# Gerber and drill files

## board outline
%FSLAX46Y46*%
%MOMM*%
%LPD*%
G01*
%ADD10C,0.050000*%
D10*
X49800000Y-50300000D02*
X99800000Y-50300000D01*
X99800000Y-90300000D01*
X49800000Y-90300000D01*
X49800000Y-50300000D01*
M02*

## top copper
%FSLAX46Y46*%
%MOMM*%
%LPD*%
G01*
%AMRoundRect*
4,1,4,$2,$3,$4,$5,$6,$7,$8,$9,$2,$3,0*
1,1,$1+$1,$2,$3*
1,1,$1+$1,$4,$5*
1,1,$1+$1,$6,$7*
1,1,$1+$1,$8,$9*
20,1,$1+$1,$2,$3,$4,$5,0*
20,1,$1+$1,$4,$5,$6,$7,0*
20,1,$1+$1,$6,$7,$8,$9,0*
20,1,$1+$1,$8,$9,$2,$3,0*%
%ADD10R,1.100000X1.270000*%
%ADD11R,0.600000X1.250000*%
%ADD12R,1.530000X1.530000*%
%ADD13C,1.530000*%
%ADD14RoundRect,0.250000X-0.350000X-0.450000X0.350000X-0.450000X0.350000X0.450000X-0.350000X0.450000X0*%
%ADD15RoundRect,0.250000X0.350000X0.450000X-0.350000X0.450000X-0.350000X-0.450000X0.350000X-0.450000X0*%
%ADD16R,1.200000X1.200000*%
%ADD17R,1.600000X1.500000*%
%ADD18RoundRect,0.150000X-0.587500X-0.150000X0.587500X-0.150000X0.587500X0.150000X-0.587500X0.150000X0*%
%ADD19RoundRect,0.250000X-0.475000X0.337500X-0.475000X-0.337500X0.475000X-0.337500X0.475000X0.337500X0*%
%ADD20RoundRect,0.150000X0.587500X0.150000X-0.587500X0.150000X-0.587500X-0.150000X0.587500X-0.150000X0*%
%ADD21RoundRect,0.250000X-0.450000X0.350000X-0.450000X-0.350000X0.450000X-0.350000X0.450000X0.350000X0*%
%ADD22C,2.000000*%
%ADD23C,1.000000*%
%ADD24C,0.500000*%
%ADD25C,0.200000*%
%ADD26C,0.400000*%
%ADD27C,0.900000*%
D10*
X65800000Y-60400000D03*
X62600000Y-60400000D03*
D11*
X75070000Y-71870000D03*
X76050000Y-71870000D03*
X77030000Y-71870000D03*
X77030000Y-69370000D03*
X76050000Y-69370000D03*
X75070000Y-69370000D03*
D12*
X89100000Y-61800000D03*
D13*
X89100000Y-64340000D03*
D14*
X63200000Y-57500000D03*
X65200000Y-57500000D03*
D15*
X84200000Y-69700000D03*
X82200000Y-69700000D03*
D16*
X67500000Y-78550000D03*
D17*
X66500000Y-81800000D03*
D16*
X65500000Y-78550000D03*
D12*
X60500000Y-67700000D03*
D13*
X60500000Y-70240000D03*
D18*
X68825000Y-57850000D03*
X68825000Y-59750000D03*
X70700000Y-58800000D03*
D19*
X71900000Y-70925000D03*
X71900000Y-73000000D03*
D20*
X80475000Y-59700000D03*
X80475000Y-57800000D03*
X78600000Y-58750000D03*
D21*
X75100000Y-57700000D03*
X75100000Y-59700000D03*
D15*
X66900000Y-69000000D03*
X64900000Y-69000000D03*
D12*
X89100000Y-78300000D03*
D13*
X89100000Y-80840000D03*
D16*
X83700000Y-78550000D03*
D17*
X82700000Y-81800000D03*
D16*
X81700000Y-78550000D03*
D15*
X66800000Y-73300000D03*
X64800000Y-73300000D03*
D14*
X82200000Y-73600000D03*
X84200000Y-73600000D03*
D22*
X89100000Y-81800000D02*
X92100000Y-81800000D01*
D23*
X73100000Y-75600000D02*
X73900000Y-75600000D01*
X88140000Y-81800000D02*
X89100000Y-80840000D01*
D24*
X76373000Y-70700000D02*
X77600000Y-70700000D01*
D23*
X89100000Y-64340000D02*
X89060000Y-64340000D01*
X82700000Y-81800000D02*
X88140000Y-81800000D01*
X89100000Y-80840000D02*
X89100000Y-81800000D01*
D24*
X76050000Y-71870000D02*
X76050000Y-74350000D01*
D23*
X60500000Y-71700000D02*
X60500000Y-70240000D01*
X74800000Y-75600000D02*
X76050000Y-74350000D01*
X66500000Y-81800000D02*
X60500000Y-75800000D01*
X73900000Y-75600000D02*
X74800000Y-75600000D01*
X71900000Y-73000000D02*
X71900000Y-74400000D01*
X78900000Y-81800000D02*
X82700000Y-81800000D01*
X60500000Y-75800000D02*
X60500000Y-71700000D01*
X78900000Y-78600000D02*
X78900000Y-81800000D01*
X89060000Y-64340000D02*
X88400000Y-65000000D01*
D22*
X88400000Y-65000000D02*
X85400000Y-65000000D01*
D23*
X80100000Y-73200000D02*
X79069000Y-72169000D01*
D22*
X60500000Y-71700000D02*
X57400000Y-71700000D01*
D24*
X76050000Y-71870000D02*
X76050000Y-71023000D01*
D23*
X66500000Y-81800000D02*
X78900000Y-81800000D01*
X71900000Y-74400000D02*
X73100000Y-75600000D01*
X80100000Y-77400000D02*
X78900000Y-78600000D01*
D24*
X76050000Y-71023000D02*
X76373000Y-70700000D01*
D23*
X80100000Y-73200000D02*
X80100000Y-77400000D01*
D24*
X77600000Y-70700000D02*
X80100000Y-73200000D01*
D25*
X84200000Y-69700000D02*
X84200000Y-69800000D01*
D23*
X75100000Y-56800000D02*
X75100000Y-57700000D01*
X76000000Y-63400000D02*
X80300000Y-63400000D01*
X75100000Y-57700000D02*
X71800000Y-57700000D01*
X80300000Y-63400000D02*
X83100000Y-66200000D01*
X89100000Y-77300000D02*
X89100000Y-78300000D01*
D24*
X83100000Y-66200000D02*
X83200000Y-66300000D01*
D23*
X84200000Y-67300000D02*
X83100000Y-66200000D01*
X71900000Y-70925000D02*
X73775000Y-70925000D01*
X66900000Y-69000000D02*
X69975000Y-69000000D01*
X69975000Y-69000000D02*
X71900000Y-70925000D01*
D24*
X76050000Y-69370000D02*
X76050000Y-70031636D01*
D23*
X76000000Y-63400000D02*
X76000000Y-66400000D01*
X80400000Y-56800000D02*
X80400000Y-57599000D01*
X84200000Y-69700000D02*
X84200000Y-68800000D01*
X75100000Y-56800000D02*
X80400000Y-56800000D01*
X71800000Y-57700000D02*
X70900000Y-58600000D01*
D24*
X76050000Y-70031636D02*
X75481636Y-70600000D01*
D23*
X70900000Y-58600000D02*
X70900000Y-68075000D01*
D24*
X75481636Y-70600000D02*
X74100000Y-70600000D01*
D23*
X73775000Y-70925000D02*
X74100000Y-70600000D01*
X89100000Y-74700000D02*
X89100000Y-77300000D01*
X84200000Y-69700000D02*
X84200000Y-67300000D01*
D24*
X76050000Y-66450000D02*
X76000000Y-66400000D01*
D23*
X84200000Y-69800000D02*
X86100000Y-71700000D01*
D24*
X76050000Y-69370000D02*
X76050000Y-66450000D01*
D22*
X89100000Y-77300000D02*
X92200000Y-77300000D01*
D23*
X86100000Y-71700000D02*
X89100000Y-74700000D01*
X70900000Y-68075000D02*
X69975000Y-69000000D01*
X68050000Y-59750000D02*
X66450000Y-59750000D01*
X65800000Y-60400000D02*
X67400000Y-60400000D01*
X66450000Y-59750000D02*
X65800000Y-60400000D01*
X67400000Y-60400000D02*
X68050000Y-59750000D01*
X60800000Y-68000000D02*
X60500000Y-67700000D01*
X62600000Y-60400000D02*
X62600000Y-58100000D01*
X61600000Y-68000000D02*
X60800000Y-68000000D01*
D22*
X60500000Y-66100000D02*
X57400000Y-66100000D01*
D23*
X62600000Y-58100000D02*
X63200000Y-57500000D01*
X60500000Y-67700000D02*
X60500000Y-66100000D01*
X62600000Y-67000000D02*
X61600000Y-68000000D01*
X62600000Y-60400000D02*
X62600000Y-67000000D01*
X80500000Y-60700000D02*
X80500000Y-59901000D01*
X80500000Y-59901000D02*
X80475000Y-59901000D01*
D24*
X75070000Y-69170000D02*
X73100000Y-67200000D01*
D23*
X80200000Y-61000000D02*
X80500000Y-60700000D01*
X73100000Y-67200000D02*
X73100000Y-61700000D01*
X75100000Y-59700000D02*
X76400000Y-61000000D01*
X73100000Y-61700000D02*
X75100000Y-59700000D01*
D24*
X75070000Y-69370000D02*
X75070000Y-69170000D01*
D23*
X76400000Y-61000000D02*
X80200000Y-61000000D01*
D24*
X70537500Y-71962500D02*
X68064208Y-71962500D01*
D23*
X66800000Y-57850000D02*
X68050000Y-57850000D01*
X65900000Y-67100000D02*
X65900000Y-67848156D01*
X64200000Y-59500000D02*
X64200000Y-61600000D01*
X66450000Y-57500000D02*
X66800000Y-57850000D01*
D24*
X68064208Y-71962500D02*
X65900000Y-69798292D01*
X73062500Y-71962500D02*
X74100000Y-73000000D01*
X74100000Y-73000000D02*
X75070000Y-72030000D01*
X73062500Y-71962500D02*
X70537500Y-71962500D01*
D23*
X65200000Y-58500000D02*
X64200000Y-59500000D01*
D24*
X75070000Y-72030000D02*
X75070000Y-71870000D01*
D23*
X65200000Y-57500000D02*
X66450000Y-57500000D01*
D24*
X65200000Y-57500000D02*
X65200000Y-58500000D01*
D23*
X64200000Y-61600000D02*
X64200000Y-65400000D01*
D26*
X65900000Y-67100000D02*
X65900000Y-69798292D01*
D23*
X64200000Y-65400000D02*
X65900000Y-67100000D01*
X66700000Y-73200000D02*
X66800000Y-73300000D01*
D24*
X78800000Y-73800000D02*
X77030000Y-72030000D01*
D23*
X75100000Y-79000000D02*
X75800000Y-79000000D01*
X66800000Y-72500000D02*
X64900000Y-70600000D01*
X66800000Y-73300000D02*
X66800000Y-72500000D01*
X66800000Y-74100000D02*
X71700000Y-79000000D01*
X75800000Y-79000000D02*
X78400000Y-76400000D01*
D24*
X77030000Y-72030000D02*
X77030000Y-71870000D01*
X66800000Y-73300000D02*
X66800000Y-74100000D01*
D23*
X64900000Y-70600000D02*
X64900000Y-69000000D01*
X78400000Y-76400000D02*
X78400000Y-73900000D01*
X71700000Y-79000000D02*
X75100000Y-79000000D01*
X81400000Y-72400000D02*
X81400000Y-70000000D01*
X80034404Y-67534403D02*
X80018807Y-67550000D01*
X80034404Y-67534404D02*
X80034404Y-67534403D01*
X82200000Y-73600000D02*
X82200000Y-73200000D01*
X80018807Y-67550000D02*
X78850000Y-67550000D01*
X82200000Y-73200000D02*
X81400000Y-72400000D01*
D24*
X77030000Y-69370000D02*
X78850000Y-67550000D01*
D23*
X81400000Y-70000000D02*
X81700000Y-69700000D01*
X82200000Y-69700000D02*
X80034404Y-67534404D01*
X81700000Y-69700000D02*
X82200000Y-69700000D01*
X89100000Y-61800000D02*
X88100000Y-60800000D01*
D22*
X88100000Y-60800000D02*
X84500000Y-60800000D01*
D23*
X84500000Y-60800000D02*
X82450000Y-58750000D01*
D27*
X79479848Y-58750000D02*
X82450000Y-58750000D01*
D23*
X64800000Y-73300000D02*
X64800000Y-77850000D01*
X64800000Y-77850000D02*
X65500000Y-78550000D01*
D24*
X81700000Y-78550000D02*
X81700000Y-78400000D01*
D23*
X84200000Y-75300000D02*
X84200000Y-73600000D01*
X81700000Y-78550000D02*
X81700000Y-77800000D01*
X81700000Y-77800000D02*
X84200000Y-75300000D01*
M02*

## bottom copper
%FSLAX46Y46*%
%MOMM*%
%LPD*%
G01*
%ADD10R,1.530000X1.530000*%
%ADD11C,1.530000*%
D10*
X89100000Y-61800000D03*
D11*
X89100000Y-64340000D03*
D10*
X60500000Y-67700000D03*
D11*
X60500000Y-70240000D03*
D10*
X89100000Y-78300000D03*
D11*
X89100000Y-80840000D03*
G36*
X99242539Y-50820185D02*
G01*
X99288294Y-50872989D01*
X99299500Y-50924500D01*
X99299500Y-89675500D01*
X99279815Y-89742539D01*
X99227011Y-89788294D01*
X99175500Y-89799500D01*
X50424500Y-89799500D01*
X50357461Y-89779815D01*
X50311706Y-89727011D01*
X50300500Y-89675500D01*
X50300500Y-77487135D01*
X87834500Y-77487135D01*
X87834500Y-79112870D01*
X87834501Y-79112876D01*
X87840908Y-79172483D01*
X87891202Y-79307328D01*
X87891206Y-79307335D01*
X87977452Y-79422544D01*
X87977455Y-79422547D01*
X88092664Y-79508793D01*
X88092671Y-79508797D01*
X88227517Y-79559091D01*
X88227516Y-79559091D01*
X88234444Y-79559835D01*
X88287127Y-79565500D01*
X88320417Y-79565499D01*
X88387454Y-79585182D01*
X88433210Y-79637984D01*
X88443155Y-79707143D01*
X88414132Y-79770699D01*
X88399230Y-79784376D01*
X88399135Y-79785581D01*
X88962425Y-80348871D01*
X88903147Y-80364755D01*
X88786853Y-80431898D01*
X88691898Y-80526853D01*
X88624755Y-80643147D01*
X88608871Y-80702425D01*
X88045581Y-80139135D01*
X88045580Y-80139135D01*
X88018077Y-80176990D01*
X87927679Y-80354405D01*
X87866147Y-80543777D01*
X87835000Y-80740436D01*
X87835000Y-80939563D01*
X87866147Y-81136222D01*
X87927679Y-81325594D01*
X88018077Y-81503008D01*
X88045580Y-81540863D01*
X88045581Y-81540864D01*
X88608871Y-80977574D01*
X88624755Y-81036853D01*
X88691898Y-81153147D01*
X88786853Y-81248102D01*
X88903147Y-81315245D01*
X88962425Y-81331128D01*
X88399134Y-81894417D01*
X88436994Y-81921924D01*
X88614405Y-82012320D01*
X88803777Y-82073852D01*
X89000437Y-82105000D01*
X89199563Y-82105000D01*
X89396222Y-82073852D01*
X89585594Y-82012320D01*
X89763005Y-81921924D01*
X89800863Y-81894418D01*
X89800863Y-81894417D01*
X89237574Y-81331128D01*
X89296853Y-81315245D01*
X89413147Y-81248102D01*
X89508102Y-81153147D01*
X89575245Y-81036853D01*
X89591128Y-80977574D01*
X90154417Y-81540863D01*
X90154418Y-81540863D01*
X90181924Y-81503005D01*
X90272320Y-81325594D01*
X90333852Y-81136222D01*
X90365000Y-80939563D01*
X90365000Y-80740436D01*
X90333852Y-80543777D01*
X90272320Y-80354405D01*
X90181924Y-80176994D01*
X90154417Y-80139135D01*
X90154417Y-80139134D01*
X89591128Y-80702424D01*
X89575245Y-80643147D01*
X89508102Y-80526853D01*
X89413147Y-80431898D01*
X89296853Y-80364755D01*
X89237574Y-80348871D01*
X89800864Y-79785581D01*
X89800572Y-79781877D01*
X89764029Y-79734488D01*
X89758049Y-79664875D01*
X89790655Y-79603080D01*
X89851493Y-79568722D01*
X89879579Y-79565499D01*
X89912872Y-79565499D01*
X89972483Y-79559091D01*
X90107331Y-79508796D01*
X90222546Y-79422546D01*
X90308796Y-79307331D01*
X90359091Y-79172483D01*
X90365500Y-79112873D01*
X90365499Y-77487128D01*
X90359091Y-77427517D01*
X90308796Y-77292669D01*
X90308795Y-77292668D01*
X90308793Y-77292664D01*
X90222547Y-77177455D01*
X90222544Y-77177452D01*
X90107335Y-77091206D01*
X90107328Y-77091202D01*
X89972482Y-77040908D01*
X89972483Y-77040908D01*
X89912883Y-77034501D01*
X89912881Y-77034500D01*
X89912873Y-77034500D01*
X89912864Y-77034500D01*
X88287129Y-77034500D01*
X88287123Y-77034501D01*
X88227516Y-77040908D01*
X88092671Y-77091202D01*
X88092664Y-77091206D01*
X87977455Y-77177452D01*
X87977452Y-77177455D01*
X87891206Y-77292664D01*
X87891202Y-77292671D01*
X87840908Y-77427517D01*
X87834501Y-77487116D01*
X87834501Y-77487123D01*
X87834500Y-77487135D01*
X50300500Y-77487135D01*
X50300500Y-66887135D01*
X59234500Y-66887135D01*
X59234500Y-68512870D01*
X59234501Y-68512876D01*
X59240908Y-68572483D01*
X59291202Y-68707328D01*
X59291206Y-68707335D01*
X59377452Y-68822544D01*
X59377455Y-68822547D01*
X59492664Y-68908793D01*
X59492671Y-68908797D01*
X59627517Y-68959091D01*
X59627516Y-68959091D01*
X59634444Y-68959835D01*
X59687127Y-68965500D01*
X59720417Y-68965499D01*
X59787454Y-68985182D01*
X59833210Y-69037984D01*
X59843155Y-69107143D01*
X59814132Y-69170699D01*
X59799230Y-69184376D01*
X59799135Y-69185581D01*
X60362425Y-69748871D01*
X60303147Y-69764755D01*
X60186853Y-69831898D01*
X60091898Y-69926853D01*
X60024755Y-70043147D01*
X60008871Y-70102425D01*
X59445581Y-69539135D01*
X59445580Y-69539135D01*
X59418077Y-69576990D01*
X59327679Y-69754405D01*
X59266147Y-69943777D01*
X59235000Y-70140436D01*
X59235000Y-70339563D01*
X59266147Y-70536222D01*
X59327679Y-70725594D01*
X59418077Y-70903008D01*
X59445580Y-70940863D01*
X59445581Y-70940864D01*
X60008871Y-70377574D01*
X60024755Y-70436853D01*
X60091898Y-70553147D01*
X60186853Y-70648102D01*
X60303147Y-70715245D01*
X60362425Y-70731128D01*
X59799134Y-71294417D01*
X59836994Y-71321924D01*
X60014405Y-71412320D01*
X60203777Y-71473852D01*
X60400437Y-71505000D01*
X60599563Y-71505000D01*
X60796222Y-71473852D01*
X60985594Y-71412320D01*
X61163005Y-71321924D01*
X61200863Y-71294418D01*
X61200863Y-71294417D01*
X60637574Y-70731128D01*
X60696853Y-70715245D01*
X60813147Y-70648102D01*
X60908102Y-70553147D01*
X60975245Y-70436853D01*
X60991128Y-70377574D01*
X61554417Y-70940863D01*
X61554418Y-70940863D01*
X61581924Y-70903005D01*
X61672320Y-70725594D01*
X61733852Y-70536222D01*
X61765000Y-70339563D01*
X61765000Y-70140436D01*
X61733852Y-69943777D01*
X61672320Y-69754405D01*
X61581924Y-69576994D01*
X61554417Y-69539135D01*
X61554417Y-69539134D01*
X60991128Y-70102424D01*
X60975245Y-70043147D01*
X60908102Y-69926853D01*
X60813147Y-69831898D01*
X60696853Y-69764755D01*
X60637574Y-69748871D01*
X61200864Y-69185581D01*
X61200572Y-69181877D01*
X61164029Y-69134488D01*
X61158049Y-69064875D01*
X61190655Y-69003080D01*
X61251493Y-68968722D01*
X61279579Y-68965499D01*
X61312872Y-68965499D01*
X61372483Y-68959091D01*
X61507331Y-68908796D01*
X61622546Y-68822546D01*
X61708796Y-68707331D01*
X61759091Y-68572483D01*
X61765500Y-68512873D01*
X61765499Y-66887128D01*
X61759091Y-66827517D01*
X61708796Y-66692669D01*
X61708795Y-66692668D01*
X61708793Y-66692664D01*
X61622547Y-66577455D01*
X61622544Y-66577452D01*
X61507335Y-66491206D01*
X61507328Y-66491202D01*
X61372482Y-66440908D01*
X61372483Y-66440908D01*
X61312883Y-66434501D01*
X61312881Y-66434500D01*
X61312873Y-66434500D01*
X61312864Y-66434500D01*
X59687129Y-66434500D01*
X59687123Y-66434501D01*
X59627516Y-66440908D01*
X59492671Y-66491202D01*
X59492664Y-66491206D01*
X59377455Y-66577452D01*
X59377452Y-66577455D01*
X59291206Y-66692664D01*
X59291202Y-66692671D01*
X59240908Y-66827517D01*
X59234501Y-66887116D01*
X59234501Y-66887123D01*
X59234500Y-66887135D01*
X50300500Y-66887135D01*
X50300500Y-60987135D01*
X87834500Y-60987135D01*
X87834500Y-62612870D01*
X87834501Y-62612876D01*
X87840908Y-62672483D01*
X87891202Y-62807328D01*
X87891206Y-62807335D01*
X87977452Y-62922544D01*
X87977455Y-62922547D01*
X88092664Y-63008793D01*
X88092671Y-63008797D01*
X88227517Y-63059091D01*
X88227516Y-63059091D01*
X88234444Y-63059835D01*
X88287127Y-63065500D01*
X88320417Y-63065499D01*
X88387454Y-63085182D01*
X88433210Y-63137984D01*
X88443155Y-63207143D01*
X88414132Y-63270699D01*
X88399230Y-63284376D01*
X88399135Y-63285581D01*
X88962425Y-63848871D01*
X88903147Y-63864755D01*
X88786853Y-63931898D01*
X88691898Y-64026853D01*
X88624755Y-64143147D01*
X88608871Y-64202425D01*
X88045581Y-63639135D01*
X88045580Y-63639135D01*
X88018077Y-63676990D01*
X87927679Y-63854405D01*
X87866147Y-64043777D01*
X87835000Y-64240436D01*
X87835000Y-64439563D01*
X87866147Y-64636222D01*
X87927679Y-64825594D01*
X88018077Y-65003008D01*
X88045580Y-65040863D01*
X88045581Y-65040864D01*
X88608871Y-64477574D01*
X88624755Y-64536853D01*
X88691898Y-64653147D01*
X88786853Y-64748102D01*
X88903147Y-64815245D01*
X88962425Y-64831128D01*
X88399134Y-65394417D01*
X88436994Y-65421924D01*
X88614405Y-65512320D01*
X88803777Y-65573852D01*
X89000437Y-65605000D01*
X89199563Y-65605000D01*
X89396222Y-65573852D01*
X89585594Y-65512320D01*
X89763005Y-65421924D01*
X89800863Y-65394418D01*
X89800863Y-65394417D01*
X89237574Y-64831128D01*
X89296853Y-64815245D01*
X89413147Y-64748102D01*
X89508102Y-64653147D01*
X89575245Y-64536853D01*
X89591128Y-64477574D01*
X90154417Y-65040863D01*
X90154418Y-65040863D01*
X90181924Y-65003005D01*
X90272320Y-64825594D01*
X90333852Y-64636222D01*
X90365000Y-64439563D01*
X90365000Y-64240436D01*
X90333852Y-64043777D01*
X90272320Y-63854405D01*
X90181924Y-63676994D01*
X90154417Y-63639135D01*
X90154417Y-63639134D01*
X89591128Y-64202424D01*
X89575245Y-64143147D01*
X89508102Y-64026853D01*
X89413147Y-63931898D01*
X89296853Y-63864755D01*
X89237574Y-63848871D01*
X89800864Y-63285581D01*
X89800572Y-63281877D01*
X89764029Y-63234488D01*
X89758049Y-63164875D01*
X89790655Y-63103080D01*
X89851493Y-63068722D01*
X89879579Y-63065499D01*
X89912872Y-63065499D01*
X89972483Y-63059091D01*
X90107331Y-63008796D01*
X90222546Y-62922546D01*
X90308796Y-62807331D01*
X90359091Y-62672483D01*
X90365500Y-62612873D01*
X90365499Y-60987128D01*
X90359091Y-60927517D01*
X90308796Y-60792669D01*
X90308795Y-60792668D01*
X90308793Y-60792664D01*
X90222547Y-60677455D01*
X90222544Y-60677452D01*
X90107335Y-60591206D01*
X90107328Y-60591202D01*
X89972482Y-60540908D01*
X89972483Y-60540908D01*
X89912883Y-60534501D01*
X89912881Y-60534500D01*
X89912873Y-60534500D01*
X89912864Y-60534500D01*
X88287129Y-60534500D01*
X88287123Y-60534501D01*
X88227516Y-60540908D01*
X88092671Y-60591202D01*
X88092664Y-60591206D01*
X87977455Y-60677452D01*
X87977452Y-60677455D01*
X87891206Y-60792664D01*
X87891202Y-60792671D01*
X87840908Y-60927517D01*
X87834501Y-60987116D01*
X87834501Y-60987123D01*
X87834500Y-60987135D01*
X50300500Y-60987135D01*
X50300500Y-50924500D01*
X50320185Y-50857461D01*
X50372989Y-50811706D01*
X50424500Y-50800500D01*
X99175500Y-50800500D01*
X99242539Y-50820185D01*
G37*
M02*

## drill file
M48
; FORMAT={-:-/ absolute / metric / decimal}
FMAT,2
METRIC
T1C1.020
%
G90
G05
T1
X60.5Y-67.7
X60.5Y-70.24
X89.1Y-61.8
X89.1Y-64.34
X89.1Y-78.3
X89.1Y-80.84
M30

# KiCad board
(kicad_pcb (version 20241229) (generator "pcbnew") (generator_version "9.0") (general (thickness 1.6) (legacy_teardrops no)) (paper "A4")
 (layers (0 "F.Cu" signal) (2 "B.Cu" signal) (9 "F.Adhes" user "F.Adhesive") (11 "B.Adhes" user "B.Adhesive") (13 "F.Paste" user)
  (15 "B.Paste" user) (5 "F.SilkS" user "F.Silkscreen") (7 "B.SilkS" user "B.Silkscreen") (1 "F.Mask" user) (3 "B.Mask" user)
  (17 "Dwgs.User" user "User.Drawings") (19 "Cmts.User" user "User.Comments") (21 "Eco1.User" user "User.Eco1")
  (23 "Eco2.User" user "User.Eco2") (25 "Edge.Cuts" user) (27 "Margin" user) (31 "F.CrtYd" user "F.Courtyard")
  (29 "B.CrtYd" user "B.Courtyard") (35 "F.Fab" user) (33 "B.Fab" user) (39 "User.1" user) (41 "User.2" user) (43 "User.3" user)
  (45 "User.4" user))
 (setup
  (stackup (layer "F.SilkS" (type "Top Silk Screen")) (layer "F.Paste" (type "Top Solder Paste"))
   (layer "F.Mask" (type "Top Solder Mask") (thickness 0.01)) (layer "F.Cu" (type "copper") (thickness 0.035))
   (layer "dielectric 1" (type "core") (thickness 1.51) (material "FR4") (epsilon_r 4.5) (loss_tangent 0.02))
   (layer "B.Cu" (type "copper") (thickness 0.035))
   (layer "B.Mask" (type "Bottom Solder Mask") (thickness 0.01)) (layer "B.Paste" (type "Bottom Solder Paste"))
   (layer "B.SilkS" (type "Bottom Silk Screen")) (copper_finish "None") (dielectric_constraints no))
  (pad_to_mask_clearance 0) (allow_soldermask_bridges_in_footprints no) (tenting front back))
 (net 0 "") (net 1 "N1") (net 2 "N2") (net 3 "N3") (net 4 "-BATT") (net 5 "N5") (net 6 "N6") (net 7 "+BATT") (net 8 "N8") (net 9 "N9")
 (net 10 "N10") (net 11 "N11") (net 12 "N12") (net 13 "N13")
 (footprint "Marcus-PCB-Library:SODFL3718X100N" (layer "F.Cu") (at 64.2 60.4 180)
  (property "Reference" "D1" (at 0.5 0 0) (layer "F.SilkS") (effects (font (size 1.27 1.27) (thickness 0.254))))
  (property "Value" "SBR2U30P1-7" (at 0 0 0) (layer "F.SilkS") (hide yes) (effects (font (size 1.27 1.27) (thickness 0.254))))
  (pad "1" smd rect (at -1.6 0 180) (size 1.1 1.27) (layers "F.Cu" "F.Mask" "F.Paste") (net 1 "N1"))
  (pad "2" smd rect (at 1.6 0 180) (size 1.1 1.27) (layers "F.Cu" "F.Mask" "F.Paste") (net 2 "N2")))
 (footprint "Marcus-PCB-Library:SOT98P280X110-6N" (layer "F.Cu") (at 76.05 70.62 90)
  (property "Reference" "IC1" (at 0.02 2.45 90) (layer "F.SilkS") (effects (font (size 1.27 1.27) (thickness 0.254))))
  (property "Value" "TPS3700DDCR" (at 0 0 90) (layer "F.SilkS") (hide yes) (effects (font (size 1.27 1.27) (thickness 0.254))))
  (pad "1" smd rect (at -1.25 -0.98 180) (size 0.6 1.25) (layers "F.Cu" "F.Mask" "F.Paste") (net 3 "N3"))
  (pad "2" smd rect (at -1.25 0 180) (size 0.6 1.25) (layers "F.Cu" "F.Mask" "F.Paste") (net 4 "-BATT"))
  (pad "3" smd rect (at -1.25 0.98 180) (size 0.6 1.25) (layers "F.Cu" "F.Mask" "F.Paste") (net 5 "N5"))
  (pad "4" smd rect (at 1.25 0.98 180) (size 0.6 1.25) (layers "F.Cu" "F.Mask" "F.Paste") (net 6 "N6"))
  (pad "5" smd rect (at 1.25 0 180) (size 0.6 1.25) (layers "F.Cu" "F.Mask" "F.Paste") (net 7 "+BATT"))
  (pad "6" smd rect (at 1.25 -0.98 180) (size 0.6 1.25) (layers "F.Cu" "F.Mask" "F.Paste") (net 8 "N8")))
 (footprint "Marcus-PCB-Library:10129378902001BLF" (layer "F.Cu") (at 89.1 61.8 -90)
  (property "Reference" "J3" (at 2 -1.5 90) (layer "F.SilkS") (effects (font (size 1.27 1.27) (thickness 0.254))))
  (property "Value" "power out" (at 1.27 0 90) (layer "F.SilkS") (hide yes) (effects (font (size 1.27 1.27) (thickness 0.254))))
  (pad "1" thru_hole rect (at 0 0 270) (size 1.53 1.53) (drill 1.02) (layers "*.Cu" "*.Mask") (remove_unused_layers no) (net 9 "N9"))
  (pad "2" thru_hole circle (at 2.54 0 270) (size 1.53 1.53) (drill 1.02) (layers "*.Cu" "*.Mask") (remove_unused_layers no) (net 4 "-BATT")))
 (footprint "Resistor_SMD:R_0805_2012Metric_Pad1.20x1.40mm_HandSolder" (layer "F.Cu") (at 64.2 57.5)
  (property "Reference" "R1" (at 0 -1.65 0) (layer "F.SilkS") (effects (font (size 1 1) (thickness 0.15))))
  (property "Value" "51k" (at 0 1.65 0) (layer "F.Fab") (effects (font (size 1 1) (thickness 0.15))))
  (pad "1" smd roundrect (at -1 0) (size 1.2 1.4) (layers "F.Cu" "F.Mask" "F.Paste") (roundrect_rratio 0.208333) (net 2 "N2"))
  (pad "2" smd roundrect (at 1 0) (size 1.2 1.4) (layers "F.Cu" "F.Mask" "F.Paste") (roundrect_rratio 0.208333) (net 3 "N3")))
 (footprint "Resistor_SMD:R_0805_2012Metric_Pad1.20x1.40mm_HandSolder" (layer "F.Cu") (at 83.2 69.7 180)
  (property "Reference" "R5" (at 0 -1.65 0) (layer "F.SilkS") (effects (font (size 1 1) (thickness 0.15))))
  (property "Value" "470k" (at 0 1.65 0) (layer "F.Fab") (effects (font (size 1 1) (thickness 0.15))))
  (pad "1" smd roundrect (at -1 0 180) (size 1.2 1.4) (layers "F.Cu" "F.Mask" "F.Paste") (roundrect_rratio 0.208333) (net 7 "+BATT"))
  (pad "2" smd roundrect (at 1 0 180) (size 1.2 1.4) (layers "F.Cu" "F.Mask" "F.Paste") (roundrect_rratio 0.208333) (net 6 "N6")))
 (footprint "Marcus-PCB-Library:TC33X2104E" (layer "F.Cu") (at 66.5 80.35 180)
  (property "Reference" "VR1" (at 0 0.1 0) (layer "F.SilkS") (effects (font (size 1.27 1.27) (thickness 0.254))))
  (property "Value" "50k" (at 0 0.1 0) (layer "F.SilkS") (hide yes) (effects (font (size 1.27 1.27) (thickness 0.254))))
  (pad "1" smd rect (at -1 1.8 270) (size 1.2 1.2) (layers "F.Cu" "F.Mask" "F.Paste") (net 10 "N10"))
  (pad "2" smd rect (at 0 -1.45 270) (size 1.5 1.6) (layers "F.Cu" "F.Mask" "F.Paste") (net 4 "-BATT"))
  (pad "3" smd rect (at 1 1.8 270) (size 1.2 1.2) (layers "F.Cu" "F.Mask" "F.Paste") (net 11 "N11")))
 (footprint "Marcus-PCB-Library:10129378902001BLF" (layer "F.Cu") (at 60.5 67.7 -90)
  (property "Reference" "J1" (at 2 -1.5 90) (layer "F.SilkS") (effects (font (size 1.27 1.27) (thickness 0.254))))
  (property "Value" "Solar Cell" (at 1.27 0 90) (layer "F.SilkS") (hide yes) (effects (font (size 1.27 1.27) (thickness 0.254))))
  (pad "1" thru_hole rect (at 0 0 270) (size 1.53 1.53) (drill 1.02) (layers "*.Cu" "*.Mask") (remove_unused_layers no) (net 2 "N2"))
  (pad "2" thru_hole circle (at 2.54 0 270) (size 1.53 1.53) (drill 1.02) (layers "*.Cu" "*.Mask") (remove_unused_layers no) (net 4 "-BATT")))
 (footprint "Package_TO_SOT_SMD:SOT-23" (layer "F.Cu") (at 69.7625 58.8)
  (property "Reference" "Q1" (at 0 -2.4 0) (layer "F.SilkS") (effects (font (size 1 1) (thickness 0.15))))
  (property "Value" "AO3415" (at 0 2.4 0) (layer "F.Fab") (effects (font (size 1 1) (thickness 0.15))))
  (pad "1" smd roundrect (at -0.9375 -0.95) (size 1.475 0.6) (layers "F.Cu" "F.Mask" "F.Paste") (roundrect_rratio 0.25) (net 3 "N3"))
  (pad "2" smd roundrect (at -0.9375 0.95) (size 1.475 0.6) (layers "F.Cu" "F.Mask" "F.Paste") (roundrect_rratio 0.25) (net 1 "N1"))
  (pad "3" smd roundrect (at 0.9375 0) (size 1.475 0.6) (layers "F.Cu" "F.Mask" "F.Paste") (roundrect_rratio 0.25) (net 7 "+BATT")))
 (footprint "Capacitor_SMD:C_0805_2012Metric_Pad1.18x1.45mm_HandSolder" (layer "F.Cu") (at 71.9 71.9625 -90)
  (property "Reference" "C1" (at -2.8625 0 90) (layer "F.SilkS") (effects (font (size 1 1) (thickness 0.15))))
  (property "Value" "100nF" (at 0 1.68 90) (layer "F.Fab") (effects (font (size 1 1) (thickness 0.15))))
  (pad "1" smd roundrect (at -1.0375 0 270) (size 1.175 1.45) (layers "F.Cu" "F.Mask" "F.Paste") (roundrect_rratio 0.212766) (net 7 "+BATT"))
  (pad "2" smd roundrect (at 1.0375 0 270) (size 1.175 1.45) (layers "F.Cu" "F.Mask" "F.Paste") (roundrect_rratio 0.212766) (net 4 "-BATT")))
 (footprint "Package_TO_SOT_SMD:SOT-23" (layer "F.Cu") (at 79.5375 58.75 180)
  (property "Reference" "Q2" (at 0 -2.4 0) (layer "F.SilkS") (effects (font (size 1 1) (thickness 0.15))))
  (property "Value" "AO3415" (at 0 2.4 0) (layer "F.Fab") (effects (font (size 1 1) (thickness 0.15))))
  (pad "1" smd roundrect (at -0.9375 -0.95 180) (size 1.475 0.6) (layers "F.Cu" "F.Mask" "F.Paste") (roundrect_rratio 0.25) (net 8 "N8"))
  (pad "2" smd roundrect (at -0.9375 0.95 180) (size 1.475 0.6) (layers "F.Cu" "F.Mask" "F.Paste") (roundrect_rratio 0.25) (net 7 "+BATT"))
  (pad "3" smd roundrect (at 0.9375 0 180) (size 1.475 0.6) (layers "F.Cu" "F.Mask" "F.Paste") (roundrect_rratio 0.25) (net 9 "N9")))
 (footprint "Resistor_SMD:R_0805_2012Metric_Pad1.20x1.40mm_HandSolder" (layer "F.Cu") (at 75.1 58.7 -90)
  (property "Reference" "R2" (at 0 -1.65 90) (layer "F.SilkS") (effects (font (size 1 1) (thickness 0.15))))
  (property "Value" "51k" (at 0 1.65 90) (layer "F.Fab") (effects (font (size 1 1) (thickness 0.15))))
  (pad "1" smd roundrect (at -1 0 270) (size 1.2 1.4) (layers "F.Cu" "F.Mask" "F.Paste") (roundrect_rratio 0.208333) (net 7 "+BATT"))
  (pad "2" smd roundrect (at 1 0 270) (size 1.2 1.4) (layers "F.Cu" "F.Mask" "F.Paste") (roundrect_rratio 0.208333) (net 8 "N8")))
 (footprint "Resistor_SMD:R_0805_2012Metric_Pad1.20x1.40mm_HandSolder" (layer "F.Cu") (at 65.9 69 180)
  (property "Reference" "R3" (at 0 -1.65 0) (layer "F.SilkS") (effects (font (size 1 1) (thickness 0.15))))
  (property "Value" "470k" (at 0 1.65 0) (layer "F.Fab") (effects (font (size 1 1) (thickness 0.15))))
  (pad "1" smd roundrect (at -1 0 180) (size 1.2 1.4) (layers "F.Cu" "F.Mask" "F.Paste") (roundrect_rratio 0.208333) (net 7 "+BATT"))
  (pad "2" smd roundrect (at 1 0 180) (size 1.2 1.4) (layers "F.Cu" "F.Mask" "F.Paste") (roundrect_rratio 0.208333) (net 5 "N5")))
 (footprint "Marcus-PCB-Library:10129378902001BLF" (layer "F.Cu") (at 89.1 78.3 -90)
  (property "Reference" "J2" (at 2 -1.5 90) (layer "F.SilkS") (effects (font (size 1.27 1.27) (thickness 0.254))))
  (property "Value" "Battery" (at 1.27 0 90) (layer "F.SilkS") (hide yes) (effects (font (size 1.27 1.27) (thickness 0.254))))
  (pad "1" thru_hole rect (at 0 0 270) (size 1.53 1.53) (drill 1.02) (layers "*.Cu" "*.Mask") (remove_unused_layers no) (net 7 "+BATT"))
  (pad "2" thru_hole circle (at 2.54 0 270) (size 1.53 1.53) (drill 1.02) (layers "*.Cu" "*.Mask") (remove_unused_layers no) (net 4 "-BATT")))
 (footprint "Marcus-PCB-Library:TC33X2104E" (layer "F.Cu") (at 82.7 80.35 180)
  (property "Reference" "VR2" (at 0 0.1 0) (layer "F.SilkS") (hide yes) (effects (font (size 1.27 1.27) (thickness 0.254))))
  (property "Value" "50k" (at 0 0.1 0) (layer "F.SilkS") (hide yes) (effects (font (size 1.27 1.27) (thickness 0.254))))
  (pad "1" smd rect (at -1 1.8 270) (size 1.2 1.2) (layers "F.Cu" "F.Mask" "F.Paste") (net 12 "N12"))
  (pad "2" smd rect (at 0 -1.45 270) (size 1.5 1.6) (layers "F.Cu" "F.Mask" "F.Paste") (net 4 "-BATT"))
  (pad "3" smd rect (at 1 1.8 270) (size 1.2 1.2) (layers "F.Cu" "F.Mask" "F.Paste") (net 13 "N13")))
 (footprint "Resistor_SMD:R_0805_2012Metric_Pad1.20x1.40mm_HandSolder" (layer "F.Cu") (at 65.8 73.3 180)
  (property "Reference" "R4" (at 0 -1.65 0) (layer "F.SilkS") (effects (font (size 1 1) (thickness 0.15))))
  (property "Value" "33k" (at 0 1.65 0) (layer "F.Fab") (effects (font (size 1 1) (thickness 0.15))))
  (pad "1" smd roundrect (at -1 0 180) (size 1.2 1.4) (layers "F.Cu" "F.Mask" "F.Paste") (roundrect_rratio 0.208333) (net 5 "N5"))
  (pad "2" smd roundrect (at 1 0 180) (size 1.2 1.4) (layers "F.Cu" "F.Mask" "F.Paste") (roundrect_rratio 0.208333) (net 11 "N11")))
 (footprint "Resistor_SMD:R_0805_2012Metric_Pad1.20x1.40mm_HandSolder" (layer "F.Cu") (at 83.2 73.6)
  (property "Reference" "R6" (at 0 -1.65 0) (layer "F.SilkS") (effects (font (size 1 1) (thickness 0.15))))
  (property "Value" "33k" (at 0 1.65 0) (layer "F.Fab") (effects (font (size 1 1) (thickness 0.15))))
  (pad "1" smd roundrect (at -1 0) (size 1.2 1.4) (layers "F.Cu" "F.Mask" "F.Paste") (roundrect_rratio 0.208333) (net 6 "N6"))
  (pad "2" smd roundrect (at 1 0) (size 1.2 1.4) (layers "F.Cu" "F.Mask" "F.Paste") (roundrect_rratio 0.208333) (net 13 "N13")))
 (gr_rect (start 49.8 50.3) (end 99.8 90.3) (stroke (width 0.05) (type default)) (fill no) (layer "Edge.Cuts"))
 (segment (start 89.1 81.8) (end 92.1 81.8) (width 2) (layer "F.Cu") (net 4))
 (segment (start 73.1 75.6) (end 73.9 75.6) (width 1) (layer "F.Cu") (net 4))
 (segment (start 88.14 81.8) (end 89.1 80.84) (width 1) (layer "F.Cu") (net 4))
 (segment (start 76.373 70.7) (end 77.6 70.7) (width 0.5) (layer "F.Cu") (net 4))
 (segment (start 89.1 64.34) (end 89.06 64.34) (width 1) (layer "F.Cu") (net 4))
 (segment (start 82.7 81.8) (end 88.14 81.8) (width 1) (layer "F.Cu") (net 4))
 (segment (start 89.1 80.84) (end 89.1 81.8) (width 1) (layer "F.Cu") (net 4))
 (segment (start 76.05 71.87) (end 76.05 74.35) (width 0.5) (layer "F.Cu") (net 4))
 (segment (start 60.5 71.7) (end 60.5 70.24) (width 1) (layer "F.Cu") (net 4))
 (segment (start 74.8 75.6) (end 76.05 74.35) (width 1) (layer "F.Cu") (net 4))
 (segment (start 66.5 81.8) (end 60.5 75.8) (width 1) (layer "F.Cu") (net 4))
 (segment (start 73.9 75.6) (end 74.8 75.6) (width 1) (layer "F.Cu") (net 4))
 (segment (start 71.9 73) (end 71.9 74.4) (width 1) (layer "F.Cu") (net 4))
 (segment (start 78.9 81.8) (end 82.7 81.8) (width 1) (layer "F.Cu") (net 4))
 (segment (start 60.5 75.8) (end 60.5 71.7) (width 1) (layer "F.Cu") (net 4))
 (segment (start 78.9 78.6) (end 78.9 81.8) (width 1) (layer "F.Cu") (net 4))
 (segment (start 89.06 64.34) (end 88.4 65) (width 1) (layer "F.Cu") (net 4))
 (segment (start 88.4 65) (end 85.4 65) (width 2) (layer "F.Cu") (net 4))
 (segment (start 80.1 73.2) (end 79.069 72.169) (width 1) (layer "F.Cu") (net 4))
 (segment (start 60.5 71.7) (end 57.4 71.7) (width 2) (layer "F.Cu") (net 4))
 (segment (start 76.05 71.87) (end 76.05 71.023) (width 0.5) (layer "F.Cu") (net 4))
 (segment (start 66.5 81.8) (end 78.9 81.8) (width 1) (layer "F.Cu") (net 4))
 (segment (start 71.9 74.4) (end 73.1 75.6) (width 1) (layer "F.Cu") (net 4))
 (segment (start 80.1 77.4) (end 78.9 78.6) (width 1) (layer "F.Cu") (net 4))
 (segment (start 76.05 71.023) (end 76.373 70.7) (width 0.5) (layer "F.Cu") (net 4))
 (segment (start 80.1 73.2) (end 80.1 77.4) (width 1) (layer "F.Cu") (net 4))
 (segment (start 77.6 70.7) (end 80.1 73.2) (width 0.5) (layer "F.Cu") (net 4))
 (segment (start 84.2 69.7) (end 84.2 69.8) (width 0.2) (layer "F.Cu") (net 7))
 (segment (start 75.1 56.8) (end 75.1 57.7) (width 1) (layer "F.Cu") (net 7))
 (segment (start 76 63.4) (end 80.3 63.4) (width 1) (layer "F.Cu") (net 7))
 (segment (start 75.1 57.7) (end 71.8 57.7) (width 1) (layer "F.Cu") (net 7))
 (segment (start 80.3 63.4) (end 83.1 66.2) (width 1) (layer "F.Cu") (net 7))
 (segment (start 89.1 77.3) (end 89.1 78.3) (width 1) (layer "F.Cu") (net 7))
 (segment (start 83.1 66.2) (end 83.2 66.3) (width 0.5) (layer "F.Cu") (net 7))
 (segment (start 84.2 67.3) (end 83.1 66.2) (width 1) (layer "F.Cu") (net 7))
 (segment (start 71.9 70.925) (end 73.775 70.925) (width 1) (layer "F.Cu") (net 7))
 (segment (start 66.9 69) (end 69.975 69) (width 1) (layer "F.Cu") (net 7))
 (segment (start 69.975 69) (end 71.9 70.925) (width 1) (layer "F.Cu") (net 7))
 (segment (start 76.05 69.37) (end 76.05 70.031636) (width 0.5) (layer "F.Cu") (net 7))
 (segment (start 76 63.4) (end 76 66.4) (width 1) (layer "F.Cu") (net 7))
 (segment (start 80.4 56.8) (end 80.4 57.599) (width 1) (layer "F.Cu") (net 7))
 (segment (start 84.2 69.7) (end 84.2 68.8) (width 1) (layer "F.Cu") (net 7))
 (segment (start 75.1 56.8) (end 80.4 56.8) (width 1) (layer "F.Cu") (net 7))
 (segment (start 71.8 57.7) (end 70.9 58.6) (width 1) (layer "F.Cu") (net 7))
 (segment (start 76.05 70.031636) (end 75.481636 70.6) (width 0.5) (layer "F.Cu") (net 7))
 (segment (start 70.9 58.6) (end 70.9 68.075) (width 1) (layer "F.Cu") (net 7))
 (segment (start 75.481636 70.6) (end 74.1 70.6) (width 0.5) (layer "F.Cu") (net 7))
 (segment (start 73.775 70.925) (end 74.1 70.6) (width 1) (layer "F.Cu") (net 7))
 (segment (start 89.1 74.7) (end 89.1 77.3) (width 1) (layer "F.Cu") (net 7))
 (segment (start 84.2 69.7) (end 84.2 67.3) (width 1) (layer "F.Cu") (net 7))
 (segment (start 76.05 66.45) (end 76 66.4) (width 0.5) (layer "F.Cu") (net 7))
 (segment (start 84.2 69.8) (end 86.1 71.7) (width 1) (layer "F.Cu") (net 7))
 (segment (start 76.05 69.37) (end 76.05 66.45) (width 0.5) (layer "F.Cu") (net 7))
 (segment (start 89.1 77.3) (end 92.2 77.3) (width 2) (layer "F.Cu") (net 7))
 (segment (start 86.1 71.7) (end 89.1 74.7) (width 1) (layer "F.Cu") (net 7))
 (segment (start 70.9 68.075) (end 69.975 69) (width 1) (layer "F.Cu") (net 7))
 (segment (start 68.05 59.75) (end 66.45 59.75) (width 1) (layer "F.Cu") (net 1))
 (segment (start 65.8 60.4) (end 67.4 60.4) (width 1) (layer "F.Cu") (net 1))
 (segment (start 66.45 59.75) (end 65.8 60.4) (width 1) (layer "F.Cu") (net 1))
 (segment (start 67.4 60.4) (end 68.05 59.75) (width 1) (layer "F.Cu") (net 1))
 (segment (start 60.8 68) (end 60.5 67.7) (width 1) (layer "F.Cu") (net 2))
 (segment (start 62.6 60.4) (end 62.6 58.1) (width 1) (layer "F.Cu") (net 2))
 (segment (start 61.6 68) (end 60.8 68) (width 1) (layer "F.Cu") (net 2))
 (segment (start 60.5 66.1) (end 57.4 66.1) (width 2) (layer "F.Cu") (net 2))
 (segment (start 62.6 58.1) (end 63.2 57.5) (width 1) (layer "F.Cu") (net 2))
 (segment (start 60.5 67.7) (end 60.5 66.1) (width 1) (layer "F.Cu") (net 2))
 (segment (start 62.6 67) (end 61.6 68) (width 1) (layer "F.Cu") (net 2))
 (segment (start 62.6 60.4) (end 62.6 67) (width 1) (layer "F.Cu") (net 2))
 (segment (start 80.5 60.7) (end 80.5 59.901) (width 1) (layer "F.Cu") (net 8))
 (segment (start 80.5 59.901) (end 80.475 59.901) (width 1) (layer "F.Cu") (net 8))
 (segment (start 75.07 69.17) (end 73.1 67.2) (width 0.5) (layer "F.Cu") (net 8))
 (segment (start 80.2 61) (end 80.5 60.7) (width 1) (layer "F.Cu") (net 8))
 (segment (start 73.1 67.2) (end 73.1 61.7) (width 1) (layer "F.Cu") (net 8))
 (segment (start 75.1 59.7) (end 76.4 61) (width 1) (layer "F.Cu") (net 8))
 (segment (start 73.1 61.7) (end 75.1 59.7) (width 1) (layer "F.Cu") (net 8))
 (segment (start 75.07 69.37) (end 75.07 69.17) (width 0.5) (layer "F.Cu") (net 8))
 (segment (start 76.4 61) (end 80.2 61) (width 1) (layer "F.Cu") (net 8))
 (segment (start 70.5375 71.9625) (end 68.064208 71.9625) (width 0.5) (layer "F.Cu") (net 3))
 (segment (start 66.8 57.85) (end 68.05 57.85) (width 1) (layer "F.Cu") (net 3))
 (segment (start 65.9 67.1) (end 65.9 67.848156) (width 1) (layer "F.Cu") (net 3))
 (segment (start 64.2 59.5) (end 64.2 61.6) (width 1) (layer "F.Cu") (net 3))
 (segment (start 66.45 57.5) (end 66.8 57.85) (width 1) (layer "F.Cu") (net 3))
 (segment (start 68.064208 71.9625) (end 65.9 69.798292) (width 0.5) (layer "F.Cu") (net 3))
 (segment (start 73.0625 71.9625) (end 74.1 73) (width 0.5) (layer "F.Cu") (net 3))
 (segment (start 74.1 73) (end 75.07 72.03) (width 0.5) (layer "F.Cu") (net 3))
 (segment (start 73.0625 71.9625) (end 70.5375 71.9625) (width 0.5) (layer "F.Cu") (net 3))
 (segment (start 65.2 58.5) (end 64.2 59.5) (width 1) (layer "F.Cu") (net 3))
 (segment (start 75.07 72.03) (end 75.07 71.87) (width 0.5) (layer "F.Cu") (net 3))
 (segment (start 65.2 57.5) (end 66.45 57.5) (width 1) (layer "F.Cu") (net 3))
 (segment (start 65.2 57.5) (end 65.2 58.5) (width 0.5) (layer "F.Cu") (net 3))
 (segment (start 64.2 61.6) (end 64.2 65.4) (width 1) (layer "F.Cu") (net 3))
 (segment (start 65.9 67.1) (end 65.9 69.798292) (width 0.4) (layer "F.Cu") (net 3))
 (segment (start 64.2 65.4) (end 65.9 67.1) (width 1) (layer "F.Cu") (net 3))
 (segment (start 66.7 73.2) (end 66.8 73.3) (width 1) (layer "F.Cu") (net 5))
 (segment (start 78.8 73.8) (end 77.03 72.03) (width 0.5) (layer "F.Cu") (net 5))
 (segment (start 75.1 79) (end 75.8 79) (width 1) (layer "F.Cu") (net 5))
 (segment (start 66.8 72.5) (end 64.9 70.6) (width 1) (layer "F.Cu") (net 5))
 (segment (start 66.8 73.3) (end 66.8 72.5) (width 1) (layer "F.Cu") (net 5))
 (segment (start 66.8 74.1) (end 71.7 79) (width 1) (layer "F.Cu") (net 5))
 (segment (start 75.8 79) (end 78.4 76.4) (width 1) (layer "F.Cu") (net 5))
 (segment (start 77.03 72.03) (end 77.03 71.87) (width 0.5) (layer "F.Cu") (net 5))
 (segment (start 66.8 73.3) (end 66.8 74.1) (width 0.5) (layer "F.Cu") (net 5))
 (segment (start 64.9 70.6) (end 64.9 69) (width 1) (layer "F.Cu") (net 5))
 (segment (start 78.4 76.4) (end 78.4 73.9) (width 1) (layer "F.Cu") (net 5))
 (segment (start 71.7 79) (end 75.1 79) (width 1) (layer "F.Cu") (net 5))
 (segment (start 81.4 72.4) (end 81.4 70) (width 1) (layer "F.Cu") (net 6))
 (segment (start 80.034404 67.534403) (end 80.018807 67.55) (width 1) (layer "F.Cu") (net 6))
 (segment (start 80.034404 67.534404) (end 80.034404 67.534403) (width 1) (layer "F.Cu") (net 6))
 (segment (start 82.2 73.6) (end 82.2 73.2) (width 1) (layer "F.Cu") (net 6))
 (segment (start 80.018807 67.55) (end 78.85 67.55) (width 1) (layer "F.Cu") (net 6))
 (segment (start 82.2 73.2) (end 81.4 72.4) (width 1) (layer "F.Cu") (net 6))
 (segment (start 77.03 69.37) (end 78.85 67.55) (width 0.5) (layer "F.Cu") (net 6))
 (segment (start 81.4 70) (end 81.7 69.7) (width 1) (layer "F.Cu") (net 6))
 (segment (start 82.2 69.7) (end 80.034404 67.534404) (width 1) (layer "F.Cu") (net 6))
 (segment (start 81.7 69.7) (end 82.2 69.7) (width 1) (layer "F.Cu") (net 6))
 (segment (start 89.1 61.8) (end 88.1 60.8) (width 1) (layer "F.Cu") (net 9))
 (segment (start 88.1 60.8) (end 84.5 60.8) (width 2) (layer "F.Cu") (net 9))
 (segment (start 84.5 60.8) (end 82.45 58.75) (width 1) (layer "F.Cu") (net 9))
 (segment (start 79.479848 58.75) (end 82.45 58.75) (width 0.9) (layer "F.Cu") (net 9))
 (segment (start 64.8 73.3) (end 64.8 77.85) (width 1) (layer "F.Cu") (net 11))
 (segment (start 64.8 77.85) (end 65.5 78.55) (width 1) (layer "F.Cu") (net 11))
 (segment (start 81.7 78.55) (end 81.7 78.4) (width 0.5) (layer "F.Cu") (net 13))
 (segment (start 84.2 75.3) (end 84.2 73.6) (width 1) (layer "F.Cu") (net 13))
 (segment (start 81.7 78.55) (end 81.7 77.8) (width 1) (layer "F.Cu") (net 13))
 (segment (start 81.7 77.8) (end 84.2 75.3) (width 1) (layer "F.Cu") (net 13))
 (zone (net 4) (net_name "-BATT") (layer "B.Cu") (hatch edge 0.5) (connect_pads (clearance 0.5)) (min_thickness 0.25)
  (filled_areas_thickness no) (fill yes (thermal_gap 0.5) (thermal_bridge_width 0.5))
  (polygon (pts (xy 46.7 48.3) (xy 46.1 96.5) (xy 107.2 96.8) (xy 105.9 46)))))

